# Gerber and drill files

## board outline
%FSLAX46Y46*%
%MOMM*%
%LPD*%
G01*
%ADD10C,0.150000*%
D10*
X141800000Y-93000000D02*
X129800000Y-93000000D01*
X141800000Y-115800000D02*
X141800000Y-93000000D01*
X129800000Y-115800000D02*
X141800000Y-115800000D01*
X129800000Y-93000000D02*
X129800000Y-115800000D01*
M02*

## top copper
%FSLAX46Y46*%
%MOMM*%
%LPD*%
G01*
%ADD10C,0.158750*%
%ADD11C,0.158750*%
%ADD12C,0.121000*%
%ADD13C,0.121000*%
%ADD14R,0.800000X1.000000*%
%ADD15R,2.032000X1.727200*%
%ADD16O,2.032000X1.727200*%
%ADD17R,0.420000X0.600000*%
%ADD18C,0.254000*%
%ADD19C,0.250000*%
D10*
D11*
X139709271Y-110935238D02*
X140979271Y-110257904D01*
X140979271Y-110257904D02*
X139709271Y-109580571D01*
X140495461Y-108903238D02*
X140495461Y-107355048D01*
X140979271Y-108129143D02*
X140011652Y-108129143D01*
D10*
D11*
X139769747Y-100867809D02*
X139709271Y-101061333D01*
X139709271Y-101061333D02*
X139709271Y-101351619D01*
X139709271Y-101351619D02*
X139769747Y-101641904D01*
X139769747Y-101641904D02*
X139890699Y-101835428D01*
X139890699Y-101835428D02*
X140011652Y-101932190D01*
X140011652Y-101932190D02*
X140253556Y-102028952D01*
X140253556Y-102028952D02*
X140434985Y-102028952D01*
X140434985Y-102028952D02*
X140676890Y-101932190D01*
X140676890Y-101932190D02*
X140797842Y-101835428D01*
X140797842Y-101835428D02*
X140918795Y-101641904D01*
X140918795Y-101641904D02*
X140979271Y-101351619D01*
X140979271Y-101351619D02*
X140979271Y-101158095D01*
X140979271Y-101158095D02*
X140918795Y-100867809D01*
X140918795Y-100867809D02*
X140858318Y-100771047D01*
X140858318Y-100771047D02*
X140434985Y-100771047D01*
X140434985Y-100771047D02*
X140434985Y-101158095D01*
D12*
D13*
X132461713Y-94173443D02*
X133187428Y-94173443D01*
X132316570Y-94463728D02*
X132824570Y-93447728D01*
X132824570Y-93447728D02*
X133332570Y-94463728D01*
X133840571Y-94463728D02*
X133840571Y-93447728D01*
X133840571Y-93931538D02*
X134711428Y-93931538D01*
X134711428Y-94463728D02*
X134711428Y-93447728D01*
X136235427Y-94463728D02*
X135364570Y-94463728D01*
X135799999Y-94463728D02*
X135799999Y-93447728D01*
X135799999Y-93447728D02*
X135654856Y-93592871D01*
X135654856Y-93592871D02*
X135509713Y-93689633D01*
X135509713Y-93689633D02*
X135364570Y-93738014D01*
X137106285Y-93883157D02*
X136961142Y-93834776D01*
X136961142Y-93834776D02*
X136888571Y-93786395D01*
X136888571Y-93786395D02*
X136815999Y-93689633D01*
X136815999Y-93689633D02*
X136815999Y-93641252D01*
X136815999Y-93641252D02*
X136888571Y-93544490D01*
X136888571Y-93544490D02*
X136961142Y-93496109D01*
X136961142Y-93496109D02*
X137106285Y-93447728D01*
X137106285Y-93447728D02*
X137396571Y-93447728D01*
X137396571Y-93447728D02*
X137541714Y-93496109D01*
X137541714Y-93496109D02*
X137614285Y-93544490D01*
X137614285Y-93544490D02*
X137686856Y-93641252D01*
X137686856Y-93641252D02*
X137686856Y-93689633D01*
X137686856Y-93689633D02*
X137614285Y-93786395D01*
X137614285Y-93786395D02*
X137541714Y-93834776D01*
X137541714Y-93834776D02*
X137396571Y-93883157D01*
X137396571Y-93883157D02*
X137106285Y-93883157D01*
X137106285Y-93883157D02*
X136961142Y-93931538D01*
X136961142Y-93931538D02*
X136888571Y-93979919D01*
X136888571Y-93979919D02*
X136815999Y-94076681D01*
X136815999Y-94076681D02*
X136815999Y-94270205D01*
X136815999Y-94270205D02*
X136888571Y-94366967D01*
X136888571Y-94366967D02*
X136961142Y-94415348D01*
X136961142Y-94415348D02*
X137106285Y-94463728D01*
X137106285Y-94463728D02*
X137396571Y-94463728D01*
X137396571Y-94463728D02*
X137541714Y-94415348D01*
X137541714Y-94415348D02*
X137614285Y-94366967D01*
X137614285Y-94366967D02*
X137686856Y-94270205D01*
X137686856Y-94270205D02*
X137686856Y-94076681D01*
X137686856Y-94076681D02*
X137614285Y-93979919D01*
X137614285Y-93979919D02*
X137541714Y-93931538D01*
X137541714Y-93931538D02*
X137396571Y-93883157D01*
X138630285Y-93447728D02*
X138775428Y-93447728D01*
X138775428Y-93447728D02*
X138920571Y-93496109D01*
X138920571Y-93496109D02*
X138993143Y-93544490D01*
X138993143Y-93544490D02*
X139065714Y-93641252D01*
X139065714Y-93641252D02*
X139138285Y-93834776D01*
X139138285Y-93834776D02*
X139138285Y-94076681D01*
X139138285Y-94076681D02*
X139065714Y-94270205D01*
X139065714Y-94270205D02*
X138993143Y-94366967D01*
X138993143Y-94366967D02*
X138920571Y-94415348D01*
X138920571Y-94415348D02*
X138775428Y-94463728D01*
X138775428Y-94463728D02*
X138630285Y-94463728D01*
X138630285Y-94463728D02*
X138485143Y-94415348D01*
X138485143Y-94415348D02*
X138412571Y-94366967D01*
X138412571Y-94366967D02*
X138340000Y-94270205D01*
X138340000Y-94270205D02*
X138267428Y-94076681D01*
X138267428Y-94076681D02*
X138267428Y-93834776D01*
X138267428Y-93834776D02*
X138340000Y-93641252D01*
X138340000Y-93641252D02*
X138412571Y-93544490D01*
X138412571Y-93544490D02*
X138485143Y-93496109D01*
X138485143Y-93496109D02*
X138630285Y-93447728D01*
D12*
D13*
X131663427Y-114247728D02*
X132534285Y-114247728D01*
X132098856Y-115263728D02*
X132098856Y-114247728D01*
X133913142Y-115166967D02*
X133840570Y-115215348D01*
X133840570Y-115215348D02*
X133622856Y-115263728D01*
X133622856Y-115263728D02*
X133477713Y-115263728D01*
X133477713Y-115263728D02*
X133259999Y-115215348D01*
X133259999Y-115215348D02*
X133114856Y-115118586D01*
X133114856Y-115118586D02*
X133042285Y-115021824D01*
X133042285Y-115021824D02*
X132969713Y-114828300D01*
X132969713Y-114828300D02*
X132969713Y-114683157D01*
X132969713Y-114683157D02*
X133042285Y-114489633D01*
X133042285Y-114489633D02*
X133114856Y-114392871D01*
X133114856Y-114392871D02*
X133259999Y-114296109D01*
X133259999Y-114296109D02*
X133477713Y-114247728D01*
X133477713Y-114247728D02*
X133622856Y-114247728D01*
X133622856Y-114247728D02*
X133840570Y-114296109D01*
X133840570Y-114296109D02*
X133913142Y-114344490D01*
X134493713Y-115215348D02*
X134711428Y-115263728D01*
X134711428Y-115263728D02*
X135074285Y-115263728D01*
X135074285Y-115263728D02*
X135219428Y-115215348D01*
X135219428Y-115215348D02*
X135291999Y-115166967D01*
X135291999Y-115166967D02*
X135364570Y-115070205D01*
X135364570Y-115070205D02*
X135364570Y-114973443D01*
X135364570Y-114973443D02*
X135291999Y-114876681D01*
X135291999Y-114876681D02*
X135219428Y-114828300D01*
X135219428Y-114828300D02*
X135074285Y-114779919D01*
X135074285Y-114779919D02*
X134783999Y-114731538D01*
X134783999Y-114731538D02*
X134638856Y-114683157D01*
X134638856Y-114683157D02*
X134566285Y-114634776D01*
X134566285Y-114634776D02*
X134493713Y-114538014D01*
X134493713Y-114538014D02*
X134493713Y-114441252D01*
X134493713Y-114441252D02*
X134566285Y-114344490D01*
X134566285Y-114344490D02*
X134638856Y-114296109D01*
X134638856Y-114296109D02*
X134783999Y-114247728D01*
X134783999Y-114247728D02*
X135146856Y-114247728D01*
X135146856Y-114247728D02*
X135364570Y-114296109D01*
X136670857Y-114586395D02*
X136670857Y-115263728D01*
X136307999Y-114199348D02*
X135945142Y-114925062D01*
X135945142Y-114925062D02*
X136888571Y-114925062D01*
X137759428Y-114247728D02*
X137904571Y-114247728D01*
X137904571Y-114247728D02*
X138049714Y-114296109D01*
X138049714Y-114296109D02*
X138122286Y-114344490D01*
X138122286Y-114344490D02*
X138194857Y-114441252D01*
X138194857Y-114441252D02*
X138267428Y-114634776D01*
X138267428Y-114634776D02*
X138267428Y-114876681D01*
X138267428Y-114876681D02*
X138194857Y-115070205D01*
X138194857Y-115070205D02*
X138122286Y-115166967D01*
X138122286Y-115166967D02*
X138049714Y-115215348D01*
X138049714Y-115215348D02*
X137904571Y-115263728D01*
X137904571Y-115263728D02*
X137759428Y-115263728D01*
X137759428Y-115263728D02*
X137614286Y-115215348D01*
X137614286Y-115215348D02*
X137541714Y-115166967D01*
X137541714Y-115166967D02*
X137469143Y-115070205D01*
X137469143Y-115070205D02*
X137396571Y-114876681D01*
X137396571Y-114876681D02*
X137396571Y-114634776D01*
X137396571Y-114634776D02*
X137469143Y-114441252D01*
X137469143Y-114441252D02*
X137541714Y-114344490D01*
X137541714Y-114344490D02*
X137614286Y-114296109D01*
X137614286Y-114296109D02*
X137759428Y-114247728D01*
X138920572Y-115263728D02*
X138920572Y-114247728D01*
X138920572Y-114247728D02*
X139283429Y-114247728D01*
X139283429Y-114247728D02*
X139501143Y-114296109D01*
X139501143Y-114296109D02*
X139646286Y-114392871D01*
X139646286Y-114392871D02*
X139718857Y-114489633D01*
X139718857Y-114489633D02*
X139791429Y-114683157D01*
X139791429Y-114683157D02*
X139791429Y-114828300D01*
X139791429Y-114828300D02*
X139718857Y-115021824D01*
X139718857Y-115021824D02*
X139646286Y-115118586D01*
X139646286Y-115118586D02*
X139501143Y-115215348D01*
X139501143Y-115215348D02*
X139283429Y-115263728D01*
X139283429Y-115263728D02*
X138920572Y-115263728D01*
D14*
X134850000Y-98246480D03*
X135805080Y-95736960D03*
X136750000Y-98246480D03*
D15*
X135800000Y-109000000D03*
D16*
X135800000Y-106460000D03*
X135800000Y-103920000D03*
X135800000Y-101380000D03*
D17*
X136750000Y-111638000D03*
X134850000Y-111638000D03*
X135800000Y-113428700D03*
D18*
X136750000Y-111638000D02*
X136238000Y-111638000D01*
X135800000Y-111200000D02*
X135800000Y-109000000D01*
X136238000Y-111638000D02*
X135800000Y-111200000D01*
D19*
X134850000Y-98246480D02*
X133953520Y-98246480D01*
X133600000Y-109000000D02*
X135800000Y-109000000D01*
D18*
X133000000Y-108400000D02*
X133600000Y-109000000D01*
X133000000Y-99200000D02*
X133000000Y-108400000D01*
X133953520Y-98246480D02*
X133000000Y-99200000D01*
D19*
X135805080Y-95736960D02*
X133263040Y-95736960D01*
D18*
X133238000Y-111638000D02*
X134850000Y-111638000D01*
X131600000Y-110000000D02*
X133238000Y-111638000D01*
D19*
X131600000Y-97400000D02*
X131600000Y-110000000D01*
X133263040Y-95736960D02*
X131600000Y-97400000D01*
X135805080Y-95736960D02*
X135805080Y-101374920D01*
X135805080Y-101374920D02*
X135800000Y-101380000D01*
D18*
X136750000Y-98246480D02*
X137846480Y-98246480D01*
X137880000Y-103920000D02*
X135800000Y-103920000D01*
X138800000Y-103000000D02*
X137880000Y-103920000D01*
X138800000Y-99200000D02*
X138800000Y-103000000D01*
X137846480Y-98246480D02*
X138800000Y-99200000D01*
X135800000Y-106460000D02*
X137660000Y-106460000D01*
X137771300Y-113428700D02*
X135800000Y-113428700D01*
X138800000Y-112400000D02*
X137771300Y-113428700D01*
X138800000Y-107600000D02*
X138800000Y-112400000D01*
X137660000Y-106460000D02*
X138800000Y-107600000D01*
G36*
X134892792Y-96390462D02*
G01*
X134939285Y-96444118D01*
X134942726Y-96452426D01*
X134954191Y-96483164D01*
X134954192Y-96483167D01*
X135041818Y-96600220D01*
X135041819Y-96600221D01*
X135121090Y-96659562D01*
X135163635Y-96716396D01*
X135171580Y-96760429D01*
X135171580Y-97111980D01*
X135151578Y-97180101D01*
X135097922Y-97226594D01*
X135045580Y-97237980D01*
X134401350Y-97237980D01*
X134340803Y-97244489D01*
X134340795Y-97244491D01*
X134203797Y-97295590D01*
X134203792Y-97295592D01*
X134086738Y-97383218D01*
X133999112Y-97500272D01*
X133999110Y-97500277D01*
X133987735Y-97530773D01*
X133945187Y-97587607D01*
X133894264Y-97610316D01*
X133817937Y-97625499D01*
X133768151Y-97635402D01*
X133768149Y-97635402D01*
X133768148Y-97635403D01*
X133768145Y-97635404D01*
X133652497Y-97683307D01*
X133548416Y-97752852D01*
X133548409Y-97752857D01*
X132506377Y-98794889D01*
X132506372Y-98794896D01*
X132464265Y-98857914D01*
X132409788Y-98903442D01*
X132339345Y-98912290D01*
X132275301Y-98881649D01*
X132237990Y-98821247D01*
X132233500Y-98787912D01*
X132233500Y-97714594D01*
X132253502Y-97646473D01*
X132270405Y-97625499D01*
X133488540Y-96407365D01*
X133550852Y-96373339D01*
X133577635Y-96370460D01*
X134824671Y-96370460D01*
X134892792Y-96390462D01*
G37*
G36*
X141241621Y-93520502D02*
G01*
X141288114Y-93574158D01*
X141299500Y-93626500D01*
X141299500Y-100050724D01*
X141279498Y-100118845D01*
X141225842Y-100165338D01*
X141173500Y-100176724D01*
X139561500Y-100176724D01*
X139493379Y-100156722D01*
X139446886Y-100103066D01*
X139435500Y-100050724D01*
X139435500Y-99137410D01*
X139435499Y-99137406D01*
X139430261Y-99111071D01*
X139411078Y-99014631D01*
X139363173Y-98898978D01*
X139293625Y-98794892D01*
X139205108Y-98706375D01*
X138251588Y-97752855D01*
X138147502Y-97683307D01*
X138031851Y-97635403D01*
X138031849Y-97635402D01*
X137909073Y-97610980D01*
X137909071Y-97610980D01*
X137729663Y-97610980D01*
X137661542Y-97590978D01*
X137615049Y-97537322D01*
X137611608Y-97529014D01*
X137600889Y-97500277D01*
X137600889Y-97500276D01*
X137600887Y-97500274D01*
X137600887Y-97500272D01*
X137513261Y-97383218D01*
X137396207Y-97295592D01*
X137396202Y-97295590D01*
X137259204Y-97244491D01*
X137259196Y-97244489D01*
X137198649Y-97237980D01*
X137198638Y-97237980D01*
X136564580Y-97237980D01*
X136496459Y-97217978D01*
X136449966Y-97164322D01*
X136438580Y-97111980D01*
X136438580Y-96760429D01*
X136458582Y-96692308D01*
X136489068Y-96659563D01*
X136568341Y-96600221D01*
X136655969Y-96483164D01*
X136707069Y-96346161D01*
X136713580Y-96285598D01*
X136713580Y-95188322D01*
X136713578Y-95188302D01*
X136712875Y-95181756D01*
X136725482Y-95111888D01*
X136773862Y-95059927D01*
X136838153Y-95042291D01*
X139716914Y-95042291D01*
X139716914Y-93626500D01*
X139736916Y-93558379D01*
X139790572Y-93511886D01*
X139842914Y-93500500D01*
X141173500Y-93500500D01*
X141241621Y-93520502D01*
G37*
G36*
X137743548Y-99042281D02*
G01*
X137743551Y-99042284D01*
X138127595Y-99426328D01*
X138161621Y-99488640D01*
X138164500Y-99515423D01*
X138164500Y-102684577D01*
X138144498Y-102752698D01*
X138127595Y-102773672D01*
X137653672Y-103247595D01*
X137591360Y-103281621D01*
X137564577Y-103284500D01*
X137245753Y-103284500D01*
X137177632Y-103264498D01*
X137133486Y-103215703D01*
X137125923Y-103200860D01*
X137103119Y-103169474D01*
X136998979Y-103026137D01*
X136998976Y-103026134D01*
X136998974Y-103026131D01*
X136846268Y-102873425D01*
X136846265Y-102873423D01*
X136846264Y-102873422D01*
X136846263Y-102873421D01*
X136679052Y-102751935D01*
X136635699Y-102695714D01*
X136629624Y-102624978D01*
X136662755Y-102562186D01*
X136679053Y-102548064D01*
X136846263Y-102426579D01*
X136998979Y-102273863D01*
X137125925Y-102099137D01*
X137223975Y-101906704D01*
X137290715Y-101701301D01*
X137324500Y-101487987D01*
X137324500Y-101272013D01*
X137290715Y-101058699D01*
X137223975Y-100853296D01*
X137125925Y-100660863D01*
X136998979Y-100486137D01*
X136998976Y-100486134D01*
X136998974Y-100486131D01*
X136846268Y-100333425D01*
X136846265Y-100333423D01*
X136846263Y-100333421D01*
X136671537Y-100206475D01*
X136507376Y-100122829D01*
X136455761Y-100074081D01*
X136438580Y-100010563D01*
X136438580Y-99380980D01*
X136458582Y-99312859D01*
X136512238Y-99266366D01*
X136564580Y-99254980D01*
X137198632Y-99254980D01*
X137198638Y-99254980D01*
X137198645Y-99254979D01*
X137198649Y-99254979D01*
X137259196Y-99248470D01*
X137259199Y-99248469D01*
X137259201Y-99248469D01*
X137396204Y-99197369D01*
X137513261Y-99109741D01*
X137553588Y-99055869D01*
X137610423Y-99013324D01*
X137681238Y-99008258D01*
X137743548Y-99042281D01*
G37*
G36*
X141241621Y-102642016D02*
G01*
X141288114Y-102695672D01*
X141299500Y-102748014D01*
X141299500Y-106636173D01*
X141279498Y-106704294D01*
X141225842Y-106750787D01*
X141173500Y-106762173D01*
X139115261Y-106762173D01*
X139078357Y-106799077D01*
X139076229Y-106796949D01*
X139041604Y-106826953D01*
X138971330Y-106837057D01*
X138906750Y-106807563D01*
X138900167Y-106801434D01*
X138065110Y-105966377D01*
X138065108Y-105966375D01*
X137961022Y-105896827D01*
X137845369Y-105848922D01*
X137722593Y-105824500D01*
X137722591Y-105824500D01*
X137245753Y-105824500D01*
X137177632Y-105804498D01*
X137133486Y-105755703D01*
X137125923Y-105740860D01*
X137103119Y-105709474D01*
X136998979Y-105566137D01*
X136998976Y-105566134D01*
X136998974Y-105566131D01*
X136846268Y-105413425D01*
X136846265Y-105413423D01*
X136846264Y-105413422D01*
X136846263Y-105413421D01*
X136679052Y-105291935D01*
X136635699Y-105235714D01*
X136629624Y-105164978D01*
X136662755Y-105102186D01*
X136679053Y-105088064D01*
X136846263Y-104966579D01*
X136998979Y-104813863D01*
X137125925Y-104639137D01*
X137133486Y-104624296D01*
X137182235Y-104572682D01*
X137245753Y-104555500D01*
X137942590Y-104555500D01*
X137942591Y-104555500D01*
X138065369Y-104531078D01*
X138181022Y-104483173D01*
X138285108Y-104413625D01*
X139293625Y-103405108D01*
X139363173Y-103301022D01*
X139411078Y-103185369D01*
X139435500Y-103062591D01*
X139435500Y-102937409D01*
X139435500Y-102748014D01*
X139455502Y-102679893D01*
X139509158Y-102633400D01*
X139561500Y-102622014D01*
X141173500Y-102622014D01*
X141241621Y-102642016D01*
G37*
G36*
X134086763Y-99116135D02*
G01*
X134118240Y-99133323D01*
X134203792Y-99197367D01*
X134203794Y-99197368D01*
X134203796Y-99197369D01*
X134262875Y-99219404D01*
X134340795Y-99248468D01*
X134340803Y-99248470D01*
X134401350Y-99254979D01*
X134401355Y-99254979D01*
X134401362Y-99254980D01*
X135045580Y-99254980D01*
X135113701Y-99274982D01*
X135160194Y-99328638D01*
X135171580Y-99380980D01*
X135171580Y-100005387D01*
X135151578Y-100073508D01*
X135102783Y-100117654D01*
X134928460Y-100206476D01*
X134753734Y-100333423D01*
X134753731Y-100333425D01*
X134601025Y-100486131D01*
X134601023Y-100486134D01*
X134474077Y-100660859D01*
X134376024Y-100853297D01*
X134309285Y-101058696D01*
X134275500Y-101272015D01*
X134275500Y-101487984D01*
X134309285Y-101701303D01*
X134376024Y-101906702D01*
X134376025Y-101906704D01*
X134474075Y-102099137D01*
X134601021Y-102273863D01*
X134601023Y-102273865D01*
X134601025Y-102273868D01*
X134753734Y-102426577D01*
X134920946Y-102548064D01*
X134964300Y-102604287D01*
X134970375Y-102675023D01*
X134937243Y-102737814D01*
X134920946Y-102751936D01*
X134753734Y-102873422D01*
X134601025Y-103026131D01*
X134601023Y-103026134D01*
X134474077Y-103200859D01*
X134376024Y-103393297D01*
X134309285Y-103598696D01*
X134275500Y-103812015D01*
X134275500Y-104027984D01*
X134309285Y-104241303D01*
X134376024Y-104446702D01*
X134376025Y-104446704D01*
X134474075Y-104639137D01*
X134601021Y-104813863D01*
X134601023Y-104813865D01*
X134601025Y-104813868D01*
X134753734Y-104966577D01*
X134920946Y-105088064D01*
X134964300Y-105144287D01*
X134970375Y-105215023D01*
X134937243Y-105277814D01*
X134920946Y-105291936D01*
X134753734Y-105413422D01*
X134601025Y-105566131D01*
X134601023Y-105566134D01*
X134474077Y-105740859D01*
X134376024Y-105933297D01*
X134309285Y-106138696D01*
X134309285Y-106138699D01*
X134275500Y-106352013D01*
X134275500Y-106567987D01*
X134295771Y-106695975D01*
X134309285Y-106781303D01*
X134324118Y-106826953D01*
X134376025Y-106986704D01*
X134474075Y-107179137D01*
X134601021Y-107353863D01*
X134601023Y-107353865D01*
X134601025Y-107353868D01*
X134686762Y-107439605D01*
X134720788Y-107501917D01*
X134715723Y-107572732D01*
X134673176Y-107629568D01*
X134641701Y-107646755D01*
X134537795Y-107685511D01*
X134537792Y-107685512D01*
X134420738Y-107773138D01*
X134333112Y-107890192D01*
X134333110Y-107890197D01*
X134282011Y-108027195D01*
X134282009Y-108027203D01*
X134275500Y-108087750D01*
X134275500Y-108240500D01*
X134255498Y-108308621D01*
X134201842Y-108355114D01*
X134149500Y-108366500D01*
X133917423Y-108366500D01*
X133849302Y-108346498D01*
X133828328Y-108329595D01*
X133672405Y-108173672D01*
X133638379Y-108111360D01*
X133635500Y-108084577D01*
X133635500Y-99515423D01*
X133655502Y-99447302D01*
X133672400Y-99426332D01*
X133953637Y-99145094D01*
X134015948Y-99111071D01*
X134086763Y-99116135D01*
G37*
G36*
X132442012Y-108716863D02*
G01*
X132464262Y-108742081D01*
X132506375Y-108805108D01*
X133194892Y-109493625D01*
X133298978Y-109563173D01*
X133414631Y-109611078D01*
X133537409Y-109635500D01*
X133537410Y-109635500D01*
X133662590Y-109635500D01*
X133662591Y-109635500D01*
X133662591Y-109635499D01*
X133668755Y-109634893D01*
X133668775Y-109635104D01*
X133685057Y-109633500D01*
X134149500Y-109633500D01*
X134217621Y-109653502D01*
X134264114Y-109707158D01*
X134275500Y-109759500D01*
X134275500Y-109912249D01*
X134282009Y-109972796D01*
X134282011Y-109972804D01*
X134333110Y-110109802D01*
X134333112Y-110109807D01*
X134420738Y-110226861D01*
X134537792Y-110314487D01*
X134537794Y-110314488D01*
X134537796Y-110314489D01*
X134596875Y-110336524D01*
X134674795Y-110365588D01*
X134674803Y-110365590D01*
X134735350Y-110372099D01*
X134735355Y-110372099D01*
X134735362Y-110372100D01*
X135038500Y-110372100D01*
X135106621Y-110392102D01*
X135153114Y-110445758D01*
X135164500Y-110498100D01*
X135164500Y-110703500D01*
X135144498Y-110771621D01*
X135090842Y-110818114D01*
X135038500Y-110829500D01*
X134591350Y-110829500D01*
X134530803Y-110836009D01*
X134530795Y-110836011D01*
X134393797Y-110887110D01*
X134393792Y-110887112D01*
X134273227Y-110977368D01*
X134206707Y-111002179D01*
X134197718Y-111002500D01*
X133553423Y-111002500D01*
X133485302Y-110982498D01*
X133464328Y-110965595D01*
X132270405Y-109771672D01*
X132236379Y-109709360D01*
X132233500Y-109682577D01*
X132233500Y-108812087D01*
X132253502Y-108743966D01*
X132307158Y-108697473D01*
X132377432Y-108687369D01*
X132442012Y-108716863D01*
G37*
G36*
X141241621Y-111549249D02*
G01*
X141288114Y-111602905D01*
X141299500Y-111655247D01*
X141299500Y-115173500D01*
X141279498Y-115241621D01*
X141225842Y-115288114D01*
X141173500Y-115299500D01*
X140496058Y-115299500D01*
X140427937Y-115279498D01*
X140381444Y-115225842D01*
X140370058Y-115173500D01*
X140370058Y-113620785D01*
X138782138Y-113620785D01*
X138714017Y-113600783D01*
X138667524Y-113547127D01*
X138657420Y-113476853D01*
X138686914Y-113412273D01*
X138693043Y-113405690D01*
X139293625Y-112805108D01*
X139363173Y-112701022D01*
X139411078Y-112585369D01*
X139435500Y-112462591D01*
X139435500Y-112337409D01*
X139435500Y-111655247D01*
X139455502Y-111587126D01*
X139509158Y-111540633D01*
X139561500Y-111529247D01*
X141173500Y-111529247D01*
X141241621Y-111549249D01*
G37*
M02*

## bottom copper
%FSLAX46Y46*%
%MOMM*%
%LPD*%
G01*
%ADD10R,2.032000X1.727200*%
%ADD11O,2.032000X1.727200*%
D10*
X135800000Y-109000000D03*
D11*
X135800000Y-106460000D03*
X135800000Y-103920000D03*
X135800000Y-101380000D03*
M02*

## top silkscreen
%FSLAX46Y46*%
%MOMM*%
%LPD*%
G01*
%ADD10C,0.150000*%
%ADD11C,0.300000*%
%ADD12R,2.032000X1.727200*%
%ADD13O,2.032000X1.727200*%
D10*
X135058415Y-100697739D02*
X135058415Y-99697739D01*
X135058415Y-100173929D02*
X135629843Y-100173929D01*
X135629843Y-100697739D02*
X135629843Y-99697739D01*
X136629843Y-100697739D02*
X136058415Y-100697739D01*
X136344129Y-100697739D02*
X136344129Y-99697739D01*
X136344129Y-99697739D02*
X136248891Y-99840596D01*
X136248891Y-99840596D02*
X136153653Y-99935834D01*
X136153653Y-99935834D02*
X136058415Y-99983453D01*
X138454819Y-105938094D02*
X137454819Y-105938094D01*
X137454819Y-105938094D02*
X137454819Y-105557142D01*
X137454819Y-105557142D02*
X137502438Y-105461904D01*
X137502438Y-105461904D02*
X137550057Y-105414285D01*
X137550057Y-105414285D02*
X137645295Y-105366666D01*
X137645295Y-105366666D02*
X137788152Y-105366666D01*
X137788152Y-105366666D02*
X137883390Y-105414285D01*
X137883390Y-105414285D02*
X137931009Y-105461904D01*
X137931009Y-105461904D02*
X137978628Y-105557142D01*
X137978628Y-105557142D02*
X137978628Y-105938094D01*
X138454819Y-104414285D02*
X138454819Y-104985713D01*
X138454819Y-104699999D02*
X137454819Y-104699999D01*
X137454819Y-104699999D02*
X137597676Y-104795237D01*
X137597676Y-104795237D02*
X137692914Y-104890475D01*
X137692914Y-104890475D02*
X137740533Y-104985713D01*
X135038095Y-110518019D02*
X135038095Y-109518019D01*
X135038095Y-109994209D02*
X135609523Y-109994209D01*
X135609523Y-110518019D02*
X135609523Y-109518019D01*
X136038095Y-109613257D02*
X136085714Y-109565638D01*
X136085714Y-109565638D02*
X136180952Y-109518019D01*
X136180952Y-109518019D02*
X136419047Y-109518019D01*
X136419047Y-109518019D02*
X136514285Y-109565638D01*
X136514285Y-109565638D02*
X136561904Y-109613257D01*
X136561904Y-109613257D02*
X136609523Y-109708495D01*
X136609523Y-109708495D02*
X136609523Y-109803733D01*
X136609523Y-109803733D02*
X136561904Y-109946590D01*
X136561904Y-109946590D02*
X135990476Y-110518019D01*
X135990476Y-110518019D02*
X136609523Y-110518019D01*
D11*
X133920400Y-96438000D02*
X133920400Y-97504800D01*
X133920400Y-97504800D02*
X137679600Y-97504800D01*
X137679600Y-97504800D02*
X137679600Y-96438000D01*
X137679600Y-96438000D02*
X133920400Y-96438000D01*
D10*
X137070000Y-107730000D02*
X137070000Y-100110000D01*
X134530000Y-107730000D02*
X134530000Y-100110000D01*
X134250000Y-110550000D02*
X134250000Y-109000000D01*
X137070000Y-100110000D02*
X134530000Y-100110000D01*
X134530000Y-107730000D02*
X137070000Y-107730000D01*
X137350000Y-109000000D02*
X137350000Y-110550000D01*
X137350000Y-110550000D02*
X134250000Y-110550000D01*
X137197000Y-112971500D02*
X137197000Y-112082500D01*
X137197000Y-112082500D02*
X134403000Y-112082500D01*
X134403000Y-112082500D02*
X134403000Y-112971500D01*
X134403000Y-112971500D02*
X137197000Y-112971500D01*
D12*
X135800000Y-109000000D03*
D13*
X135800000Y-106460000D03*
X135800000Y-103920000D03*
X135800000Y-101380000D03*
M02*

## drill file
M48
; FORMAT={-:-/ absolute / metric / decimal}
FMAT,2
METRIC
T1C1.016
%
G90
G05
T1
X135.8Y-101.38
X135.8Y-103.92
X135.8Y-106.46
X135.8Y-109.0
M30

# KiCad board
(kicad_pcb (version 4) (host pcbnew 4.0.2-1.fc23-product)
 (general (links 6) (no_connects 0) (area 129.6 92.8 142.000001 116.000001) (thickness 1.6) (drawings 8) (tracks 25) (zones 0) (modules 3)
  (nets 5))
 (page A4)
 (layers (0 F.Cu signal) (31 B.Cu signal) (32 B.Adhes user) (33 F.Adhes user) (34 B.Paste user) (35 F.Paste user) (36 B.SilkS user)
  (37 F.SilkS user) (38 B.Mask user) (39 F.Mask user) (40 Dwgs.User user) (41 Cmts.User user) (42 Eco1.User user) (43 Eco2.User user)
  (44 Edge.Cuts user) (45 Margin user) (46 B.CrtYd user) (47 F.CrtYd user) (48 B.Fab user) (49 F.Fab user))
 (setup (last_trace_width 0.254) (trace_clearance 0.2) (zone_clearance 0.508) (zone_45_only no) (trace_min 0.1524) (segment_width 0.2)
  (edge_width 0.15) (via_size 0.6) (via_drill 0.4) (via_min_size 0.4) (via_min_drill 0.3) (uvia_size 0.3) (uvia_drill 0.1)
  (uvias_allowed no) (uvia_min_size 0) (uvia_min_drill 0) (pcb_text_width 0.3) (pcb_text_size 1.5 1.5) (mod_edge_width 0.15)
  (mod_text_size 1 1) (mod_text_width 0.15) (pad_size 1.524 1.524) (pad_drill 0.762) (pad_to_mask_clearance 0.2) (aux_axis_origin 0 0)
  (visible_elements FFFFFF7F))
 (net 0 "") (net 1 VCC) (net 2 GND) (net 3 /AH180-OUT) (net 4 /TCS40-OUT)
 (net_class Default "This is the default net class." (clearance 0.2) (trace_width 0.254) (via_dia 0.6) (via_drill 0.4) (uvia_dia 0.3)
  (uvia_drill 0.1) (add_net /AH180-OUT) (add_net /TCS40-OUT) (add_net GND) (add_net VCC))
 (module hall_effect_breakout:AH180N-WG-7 (layer F.Cu) (at 135.8 97.2)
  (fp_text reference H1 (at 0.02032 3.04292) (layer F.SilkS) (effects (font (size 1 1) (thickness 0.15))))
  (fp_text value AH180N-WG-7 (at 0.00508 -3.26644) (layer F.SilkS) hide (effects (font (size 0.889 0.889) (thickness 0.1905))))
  (fp_line (start -1.8796 -0.762) (end -1.8796 0.3048) (layer F.SilkS) (width 0.3))
  (fp_line (start -1.8796 0.3048) (end 1.8796 0.3048) (layer F.SilkS) (width 0.3))
  (fp_line (start 1.8796 0.3048) (end 1.8796 -0.762) (layer F.SilkS) (width 0.3))
  (fp_line (start 1.8796 -0.762) (end -1.8796 -0.762) (layer F.SilkS) (width 0.3))
  (pad 1 smd rect (at -0.95 1.04648) (size 0.8 1) (layers F.Cu F.Paste F.Mask) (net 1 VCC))
  (pad 2 smd rect (at 0.00508 -1.46304) (size 0.8 1) (layers F.Cu F.Paste F.Mask) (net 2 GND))
  (pad 3 smd rect (at 0.95 1.04648) (size 0.8 1) (layers F.Cu F.Paste F.Mask) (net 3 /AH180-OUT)))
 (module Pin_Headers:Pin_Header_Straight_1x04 (layer F.Cu) (at 135.8 109 180)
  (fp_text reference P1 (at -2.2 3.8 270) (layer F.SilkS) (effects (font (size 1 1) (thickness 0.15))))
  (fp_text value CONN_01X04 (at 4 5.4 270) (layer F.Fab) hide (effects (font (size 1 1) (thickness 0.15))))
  (fp_line (start -1.27 1.27) (end -1.27 8.89) (layer F.SilkS) (width 0.15))
  (fp_line (start 1.27 1.27) (end 1.27 8.89) (layer F.SilkS) (width 0.15))
  (fp_line (start 1.55 -1.55) (end 1.55 0) (layer F.SilkS) (width 0.15))
  (fp_line (start -1.27 8.89) (end 1.27 8.89) (layer F.SilkS) (width 0.15))
  (fp_line (start 1.27 1.27) (end -1.27 1.27) (layer F.SilkS) (width 0.15))
  (fp_line (start -1.55 0) (end -1.55 -1.55) (layer F.SilkS) (width 0.15))
  (fp_line (start -1.55 -1.55) (end 1.55 -1.55) (layer F.SilkS) (width 0.15))
  (pad 1 thru_hole rect (at 0 0 180) (size 2.032 1.7272) (drill 1.016) (layers *.Cu *.Mask F.SilkS) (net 1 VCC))
  (pad 2 thru_hole oval (at 0 2.54 180) (size 2.032 1.7272) (drill 1.016) (layers *.Cu *.Mask F.SilkS) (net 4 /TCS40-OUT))
  (pad 3 thru_hole oval (at 0 5.08 180) (size 2.032 1.7272) (drill 1.016) (layers *.Cu *.Mask F.SilkS) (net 3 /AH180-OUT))
  (pad 4 thru_hole oval (at 0 7.62 180) (size 2.032 1.7272) (drill 1.016) (layers *.Cu *.Mask F.SilkS) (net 2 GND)))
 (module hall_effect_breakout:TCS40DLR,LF (layer F.Cu) (at 135.8 112.4 180)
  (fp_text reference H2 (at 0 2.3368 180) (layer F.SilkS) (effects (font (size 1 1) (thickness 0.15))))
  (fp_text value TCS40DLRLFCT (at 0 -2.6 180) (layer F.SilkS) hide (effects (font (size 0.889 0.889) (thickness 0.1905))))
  (fp_line (start -1.397 -0.5715) (end -1.397 0.3175) (layer F.SilkS) (width 0.15))
  (fp_line (start -1.397 0.3175) (end 1.397 0.3175) (layer F.SilkS) (width 0.15))
  (fp_line (start 1.397 0.3175) (end 1.397 -0.5715) (layer F.SilkS) (width 0.15))
  (fp_line (start 1.397 -0.5715) (end -1.397 -0.5715) (layer F.SilkS) (width 0.15))
  (pad 1 smd rect (at -0.95 0.762 180) (size 0.42 0.6) (layers F.Cu F.Paste F.Mask) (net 1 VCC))
  (pad 2 smd rect (at 0.95 0.762 180) (size 0.42 0.6) (layers F.Cu F.Paste F.Mask) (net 2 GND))
  (pad 3 smd rect (at 0 -1.0287 180) (size 0.42 0.6) (layers F.Cu F.Paste F.Mask) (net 4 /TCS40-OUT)))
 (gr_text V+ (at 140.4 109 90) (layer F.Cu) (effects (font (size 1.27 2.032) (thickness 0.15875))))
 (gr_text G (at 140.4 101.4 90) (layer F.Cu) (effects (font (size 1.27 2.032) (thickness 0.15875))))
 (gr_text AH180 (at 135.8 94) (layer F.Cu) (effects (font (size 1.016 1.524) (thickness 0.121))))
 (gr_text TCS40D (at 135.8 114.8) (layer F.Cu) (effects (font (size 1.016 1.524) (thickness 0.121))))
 (gr_line (start 141.8 93) (end 129.8 93) (angle 90) (layer Edge.Cuts) (width 0.15))
 (gr_line (start 141.8 115.8) (end 141.8 93) (angle 90) (layer Edge.Cuts) (width 0.15))
 (gr_line (start 129.8 115.8) (end 141.8 115.8) (angle 90) (layer Edge.Cuts) (width 0.15))
 (gr_line (start 129.8 93) (end 129.8 115.8) (angle 90) (layer Edge.Cuts) (width 0.15))
 (segment (start 136.75 111.638) (end 136.238 111.638) (width 0.254) (layer F.Cu) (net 1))
 (segment (start 135.8 111.2) (end 135.8 109) (width 0.254) (layer F.Cu) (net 1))
 (segment (start 136.238 111.638) (end 135.8 111.2) (width 0.254) (layer F.Cu) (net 1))
 (segment (start 134.85 98.24648) (end 133.95352 98.24648) (width 0.25) (layer F.Cu) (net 1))
 (segment (start 133.6 109) (end 135.8 109) (width 0.25) (layer F.Cu) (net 1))
 (segment (start 133 108.4) (end 133.6 109) (width 0.254) (layer F.Cu) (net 1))
 (segment (start 133 99.2) (end 133 108.4) (width 0.254) (layer F.Cu) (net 1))
 (segment (start 133.95352 98.24648) (end 133 99.2) (width 0.254) (layer F.Cu) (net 1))
 (segment (start 135.80508 95.73696) (end 133.26304 95.73696) (width 0.25) (layer F.Cu) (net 2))
 (segment (start 133.238 111.638) (end 134.85 111.638) (width 0.254) (layer F.Cu) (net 2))
 (segment (start 131.6 110) (end 133.238 111.638) (width 0.254) (layer F.Cu) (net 2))
 (segment (start 131.6 97.4) (end 131.6 110) (width 0.25) (layer F.Cu) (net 2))
 (segment (start 133.26304 95.73696) (end 131.6 97.4) (width 0.25) (layer F.Cu) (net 2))
 (segment (start 135.80508 95.73696) (end 135.80508 101.37492) (width 0.25) (layer F.Cu) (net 2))
 (segment (start 135.80508 101.37492) (end 135.8 101.38) (width 0.25) (layer F.Cu) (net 2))
 (segment (start 136.75 98.24648) (end 137.84648 98.24648) (width 0.254) (layer F.Cu) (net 3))
 (segment (start 137.88 103.92) (end 135.8 103.92) (width 0.254) (layer F.Cu) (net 3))
 (segment (start 138.8 103) (end 137.88 103.92) (width 0.254) (layer F.Cu) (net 3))
 (segment (start 138.8 99.2) (end 138.8 103) (width 0.254) (layer F.Cu) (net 3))
 (segment (start 137.84648 98.24648) (end 138.8 99.2) (width 0.254) (layer F.Cu) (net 3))
 (segment (start 135.8 106.46) (end 137.66 106.46) (width 0.254) (layer F.Cu) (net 4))
 (segment (start 137.7713 113.4287) (end 135.8 113.4287) (width 0.254) (layer F.Cu) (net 4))
 (segment (start 138.8 112.4) (end 137.7713 113.4287) (width 0.254) (layer F.Cu) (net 4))
 (segment (start 138.8 107.6) (end 138.8 112.4) (width 0.254) (layer F.Cu) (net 4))
 (segment (start 137.66 106.46) (end 138.8 107.6) (width 0.254) (layer F.Cu) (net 4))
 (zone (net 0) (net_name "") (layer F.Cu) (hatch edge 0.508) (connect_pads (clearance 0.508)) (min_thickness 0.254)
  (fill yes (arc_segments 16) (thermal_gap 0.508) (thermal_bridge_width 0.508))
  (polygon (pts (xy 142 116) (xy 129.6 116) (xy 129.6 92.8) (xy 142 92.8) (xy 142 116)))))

